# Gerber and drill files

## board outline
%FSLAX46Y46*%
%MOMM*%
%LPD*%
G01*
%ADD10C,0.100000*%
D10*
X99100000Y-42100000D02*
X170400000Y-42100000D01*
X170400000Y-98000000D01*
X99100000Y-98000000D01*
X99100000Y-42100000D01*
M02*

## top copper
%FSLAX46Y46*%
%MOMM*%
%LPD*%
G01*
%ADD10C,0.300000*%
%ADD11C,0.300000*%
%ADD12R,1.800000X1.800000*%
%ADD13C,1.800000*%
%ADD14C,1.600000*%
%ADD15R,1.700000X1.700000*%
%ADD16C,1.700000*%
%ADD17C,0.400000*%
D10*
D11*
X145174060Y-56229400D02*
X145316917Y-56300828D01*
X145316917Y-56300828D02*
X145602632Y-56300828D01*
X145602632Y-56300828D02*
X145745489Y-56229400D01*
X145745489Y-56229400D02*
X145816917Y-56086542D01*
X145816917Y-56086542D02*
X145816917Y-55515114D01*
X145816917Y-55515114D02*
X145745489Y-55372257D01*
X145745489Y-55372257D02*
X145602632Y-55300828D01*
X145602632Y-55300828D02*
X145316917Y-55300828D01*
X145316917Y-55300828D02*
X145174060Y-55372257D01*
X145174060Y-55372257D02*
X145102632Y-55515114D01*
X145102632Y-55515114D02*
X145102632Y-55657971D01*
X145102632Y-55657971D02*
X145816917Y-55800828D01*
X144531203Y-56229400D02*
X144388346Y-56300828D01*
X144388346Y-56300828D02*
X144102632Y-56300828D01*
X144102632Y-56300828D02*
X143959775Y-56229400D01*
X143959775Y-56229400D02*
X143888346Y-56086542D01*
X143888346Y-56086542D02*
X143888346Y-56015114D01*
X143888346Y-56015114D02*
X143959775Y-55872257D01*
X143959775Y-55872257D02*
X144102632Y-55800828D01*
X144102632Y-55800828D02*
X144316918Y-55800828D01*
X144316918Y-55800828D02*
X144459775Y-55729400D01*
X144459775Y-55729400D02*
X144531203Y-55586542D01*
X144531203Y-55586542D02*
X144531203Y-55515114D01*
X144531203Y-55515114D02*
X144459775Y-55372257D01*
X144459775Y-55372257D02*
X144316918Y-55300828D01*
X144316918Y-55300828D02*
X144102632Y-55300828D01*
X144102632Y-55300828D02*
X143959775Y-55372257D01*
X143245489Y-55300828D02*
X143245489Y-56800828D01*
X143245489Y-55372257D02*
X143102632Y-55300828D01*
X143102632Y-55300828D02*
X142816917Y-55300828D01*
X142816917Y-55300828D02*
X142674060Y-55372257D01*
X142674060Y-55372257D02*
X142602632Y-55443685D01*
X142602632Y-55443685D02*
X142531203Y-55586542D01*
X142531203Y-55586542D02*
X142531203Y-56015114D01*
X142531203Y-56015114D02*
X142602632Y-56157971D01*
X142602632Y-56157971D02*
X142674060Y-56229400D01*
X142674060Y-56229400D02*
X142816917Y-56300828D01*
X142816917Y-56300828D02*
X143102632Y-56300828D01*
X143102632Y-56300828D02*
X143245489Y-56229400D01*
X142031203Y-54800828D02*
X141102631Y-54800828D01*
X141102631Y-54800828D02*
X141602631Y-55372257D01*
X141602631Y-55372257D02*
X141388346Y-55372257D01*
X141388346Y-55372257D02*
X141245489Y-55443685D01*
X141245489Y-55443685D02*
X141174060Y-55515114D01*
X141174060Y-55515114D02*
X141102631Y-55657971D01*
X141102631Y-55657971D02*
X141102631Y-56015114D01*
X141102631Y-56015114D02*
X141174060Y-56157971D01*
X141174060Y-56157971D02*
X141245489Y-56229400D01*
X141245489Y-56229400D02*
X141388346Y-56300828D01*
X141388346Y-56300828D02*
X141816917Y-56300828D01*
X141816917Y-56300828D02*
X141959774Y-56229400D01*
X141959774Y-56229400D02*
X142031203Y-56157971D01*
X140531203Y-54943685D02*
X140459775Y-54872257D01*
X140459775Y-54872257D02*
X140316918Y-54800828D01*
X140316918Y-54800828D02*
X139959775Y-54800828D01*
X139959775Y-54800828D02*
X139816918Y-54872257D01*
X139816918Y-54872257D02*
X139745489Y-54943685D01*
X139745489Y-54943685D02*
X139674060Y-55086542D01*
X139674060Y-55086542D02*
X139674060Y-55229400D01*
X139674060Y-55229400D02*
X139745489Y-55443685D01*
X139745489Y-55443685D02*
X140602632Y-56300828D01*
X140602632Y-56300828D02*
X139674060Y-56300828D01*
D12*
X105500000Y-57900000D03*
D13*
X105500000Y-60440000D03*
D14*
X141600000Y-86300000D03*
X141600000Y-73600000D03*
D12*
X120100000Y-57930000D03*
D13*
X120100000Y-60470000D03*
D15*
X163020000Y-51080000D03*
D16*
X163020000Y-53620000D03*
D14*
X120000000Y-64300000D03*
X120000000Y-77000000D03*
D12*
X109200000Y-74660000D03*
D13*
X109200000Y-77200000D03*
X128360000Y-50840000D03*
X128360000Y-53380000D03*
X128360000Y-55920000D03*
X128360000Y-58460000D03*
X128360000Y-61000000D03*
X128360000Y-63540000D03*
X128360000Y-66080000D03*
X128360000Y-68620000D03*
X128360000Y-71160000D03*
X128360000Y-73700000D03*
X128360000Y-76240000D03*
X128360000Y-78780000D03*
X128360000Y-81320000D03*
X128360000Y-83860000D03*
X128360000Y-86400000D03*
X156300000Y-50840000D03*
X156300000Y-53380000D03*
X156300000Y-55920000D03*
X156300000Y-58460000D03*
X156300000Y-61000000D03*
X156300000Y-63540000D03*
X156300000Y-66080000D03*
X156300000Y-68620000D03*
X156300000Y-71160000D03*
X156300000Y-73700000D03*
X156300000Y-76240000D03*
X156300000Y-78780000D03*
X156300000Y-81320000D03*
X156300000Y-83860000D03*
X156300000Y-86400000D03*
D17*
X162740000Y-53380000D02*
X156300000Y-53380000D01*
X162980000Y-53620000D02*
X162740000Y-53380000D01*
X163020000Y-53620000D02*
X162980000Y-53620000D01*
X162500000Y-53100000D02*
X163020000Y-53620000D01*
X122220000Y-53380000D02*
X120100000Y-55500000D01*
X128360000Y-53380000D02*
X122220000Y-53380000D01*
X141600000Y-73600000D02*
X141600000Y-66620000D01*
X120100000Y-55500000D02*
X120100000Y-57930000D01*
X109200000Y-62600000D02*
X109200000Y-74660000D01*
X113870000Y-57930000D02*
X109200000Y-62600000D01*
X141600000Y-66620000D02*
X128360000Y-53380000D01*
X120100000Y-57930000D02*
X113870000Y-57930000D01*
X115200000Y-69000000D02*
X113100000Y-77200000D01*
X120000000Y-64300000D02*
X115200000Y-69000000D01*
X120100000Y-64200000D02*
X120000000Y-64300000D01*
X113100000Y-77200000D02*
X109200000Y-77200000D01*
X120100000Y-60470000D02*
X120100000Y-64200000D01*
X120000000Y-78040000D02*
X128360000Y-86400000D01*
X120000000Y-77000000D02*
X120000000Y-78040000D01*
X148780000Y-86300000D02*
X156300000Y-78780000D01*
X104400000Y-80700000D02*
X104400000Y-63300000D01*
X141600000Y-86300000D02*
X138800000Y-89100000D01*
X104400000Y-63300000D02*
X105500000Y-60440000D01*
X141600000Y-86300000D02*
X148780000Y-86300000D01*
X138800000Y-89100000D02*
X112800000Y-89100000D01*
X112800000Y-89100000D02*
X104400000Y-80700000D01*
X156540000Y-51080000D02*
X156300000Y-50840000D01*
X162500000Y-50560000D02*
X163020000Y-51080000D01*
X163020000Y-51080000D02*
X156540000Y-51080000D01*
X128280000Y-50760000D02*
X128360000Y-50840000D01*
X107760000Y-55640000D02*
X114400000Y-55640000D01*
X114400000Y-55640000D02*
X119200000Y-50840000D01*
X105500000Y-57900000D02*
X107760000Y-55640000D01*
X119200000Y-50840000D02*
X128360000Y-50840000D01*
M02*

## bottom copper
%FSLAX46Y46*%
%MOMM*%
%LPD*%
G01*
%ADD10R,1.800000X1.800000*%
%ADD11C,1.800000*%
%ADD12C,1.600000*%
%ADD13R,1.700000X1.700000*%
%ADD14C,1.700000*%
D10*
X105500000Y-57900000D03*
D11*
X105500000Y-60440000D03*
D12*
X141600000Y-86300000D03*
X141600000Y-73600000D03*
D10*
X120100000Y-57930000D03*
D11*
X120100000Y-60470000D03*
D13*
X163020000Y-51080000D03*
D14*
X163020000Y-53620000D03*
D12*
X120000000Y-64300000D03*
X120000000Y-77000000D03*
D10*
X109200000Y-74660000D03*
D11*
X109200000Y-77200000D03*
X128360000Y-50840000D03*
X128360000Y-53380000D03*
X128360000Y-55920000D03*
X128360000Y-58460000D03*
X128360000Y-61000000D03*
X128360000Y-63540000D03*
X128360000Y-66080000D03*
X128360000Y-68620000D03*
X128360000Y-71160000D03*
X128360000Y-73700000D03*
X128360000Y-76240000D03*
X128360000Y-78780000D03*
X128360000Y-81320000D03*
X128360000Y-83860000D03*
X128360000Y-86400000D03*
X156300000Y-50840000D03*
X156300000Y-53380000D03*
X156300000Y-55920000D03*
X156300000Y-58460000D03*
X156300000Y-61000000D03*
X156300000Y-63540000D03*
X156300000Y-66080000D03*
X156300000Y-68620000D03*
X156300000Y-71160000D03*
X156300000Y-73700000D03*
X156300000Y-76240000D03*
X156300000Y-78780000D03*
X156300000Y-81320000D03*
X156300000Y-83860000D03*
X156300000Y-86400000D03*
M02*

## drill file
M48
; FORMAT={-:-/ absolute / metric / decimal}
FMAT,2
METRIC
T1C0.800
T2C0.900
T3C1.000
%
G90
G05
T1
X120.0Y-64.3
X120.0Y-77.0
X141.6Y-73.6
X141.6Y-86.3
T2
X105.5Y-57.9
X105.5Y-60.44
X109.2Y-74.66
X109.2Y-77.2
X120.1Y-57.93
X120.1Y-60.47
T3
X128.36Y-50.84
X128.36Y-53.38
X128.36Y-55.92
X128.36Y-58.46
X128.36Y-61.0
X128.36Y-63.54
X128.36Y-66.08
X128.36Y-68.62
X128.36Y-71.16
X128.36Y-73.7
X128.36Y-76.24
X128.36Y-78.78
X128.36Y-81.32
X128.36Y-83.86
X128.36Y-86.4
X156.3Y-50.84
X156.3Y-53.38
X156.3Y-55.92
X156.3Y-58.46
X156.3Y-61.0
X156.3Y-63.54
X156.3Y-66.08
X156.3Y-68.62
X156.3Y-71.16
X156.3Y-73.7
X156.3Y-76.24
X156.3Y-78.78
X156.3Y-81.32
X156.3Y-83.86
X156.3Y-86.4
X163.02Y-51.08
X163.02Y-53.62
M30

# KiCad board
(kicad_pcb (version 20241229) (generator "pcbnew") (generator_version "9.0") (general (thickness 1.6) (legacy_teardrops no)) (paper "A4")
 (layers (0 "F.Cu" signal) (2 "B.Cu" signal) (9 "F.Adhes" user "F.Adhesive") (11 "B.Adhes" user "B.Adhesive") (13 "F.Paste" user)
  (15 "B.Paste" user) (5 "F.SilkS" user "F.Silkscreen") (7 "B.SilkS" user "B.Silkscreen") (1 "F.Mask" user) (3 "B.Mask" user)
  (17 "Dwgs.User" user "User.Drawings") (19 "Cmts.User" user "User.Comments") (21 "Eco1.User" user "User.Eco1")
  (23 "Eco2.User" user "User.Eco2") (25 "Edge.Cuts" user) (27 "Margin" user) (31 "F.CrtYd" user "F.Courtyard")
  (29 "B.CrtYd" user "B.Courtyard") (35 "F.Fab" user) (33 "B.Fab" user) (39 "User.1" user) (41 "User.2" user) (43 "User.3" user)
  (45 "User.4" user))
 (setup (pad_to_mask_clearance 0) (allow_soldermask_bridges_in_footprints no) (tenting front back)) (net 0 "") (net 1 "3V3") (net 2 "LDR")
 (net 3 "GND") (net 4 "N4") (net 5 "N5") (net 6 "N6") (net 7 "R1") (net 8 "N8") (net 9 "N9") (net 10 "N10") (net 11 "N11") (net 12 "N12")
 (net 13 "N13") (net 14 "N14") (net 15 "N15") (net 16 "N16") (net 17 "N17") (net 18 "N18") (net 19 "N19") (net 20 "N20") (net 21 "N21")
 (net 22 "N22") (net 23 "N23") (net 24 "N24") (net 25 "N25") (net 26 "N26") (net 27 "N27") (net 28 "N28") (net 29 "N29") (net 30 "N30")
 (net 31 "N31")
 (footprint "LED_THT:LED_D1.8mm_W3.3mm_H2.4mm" (layer "F.Cu") (at 105.5 57.9 -90)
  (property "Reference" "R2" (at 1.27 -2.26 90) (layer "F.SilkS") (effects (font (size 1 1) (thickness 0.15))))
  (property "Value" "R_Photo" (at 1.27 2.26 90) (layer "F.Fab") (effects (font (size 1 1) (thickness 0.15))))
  (pad "1" thru_hole rect (at 0 0 270) (size 1.8 1.8) (drill 0.9) (layers "*.Cu" "*.Mask") (remove_unused_layers no) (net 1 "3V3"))
  (pad "2" thru_hole circle (at 2.54 0 270) (size 1.8 1.8) (drill 0.9) (layers "*.Cu" "*.Mask") (remove_unused_layers no) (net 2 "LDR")))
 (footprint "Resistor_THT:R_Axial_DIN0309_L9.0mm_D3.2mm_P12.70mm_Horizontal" (layer "F.Cu") (at 141.6 86.3 90)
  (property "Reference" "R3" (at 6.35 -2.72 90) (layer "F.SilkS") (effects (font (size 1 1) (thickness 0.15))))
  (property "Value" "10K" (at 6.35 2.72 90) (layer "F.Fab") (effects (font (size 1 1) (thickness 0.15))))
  (pad "1" thru_hole circle (at 0 0 90) (size 1.6 1.6) (drill 0.8) (layers "*.Cu" "*.Mask") (remove_unused_layers no) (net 2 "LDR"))
  (pad "2" thru_hole circle (at 12.7 0 90) (size 1.6 1.6) (drill 0.8) (layers "*.Cu" "*.Mask") (remove_unused_layers no) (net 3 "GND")))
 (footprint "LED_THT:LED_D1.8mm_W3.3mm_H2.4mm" (layer "F.Cu") (at 120.1 57.93 -90)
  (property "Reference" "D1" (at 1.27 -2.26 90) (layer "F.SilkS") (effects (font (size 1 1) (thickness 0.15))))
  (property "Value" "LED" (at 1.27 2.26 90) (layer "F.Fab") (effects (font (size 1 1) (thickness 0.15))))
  (pad "1" thru_hole rect (at 0 0 270) (size 1.8 1.8) (drill 0.9) (layers "*.Cu" "*.Mask") (remove_unused_layers no) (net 3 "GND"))
  (pad "2" thru_hole circle (at 2.54 0 270) (size 1.8 1.8) (drill 0.9) (layers "*.Cu" "*.Mask") (remove_unused_layers no) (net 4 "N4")))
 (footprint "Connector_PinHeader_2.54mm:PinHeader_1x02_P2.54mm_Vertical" (layer "F.Cu") (at 163.02 51.08)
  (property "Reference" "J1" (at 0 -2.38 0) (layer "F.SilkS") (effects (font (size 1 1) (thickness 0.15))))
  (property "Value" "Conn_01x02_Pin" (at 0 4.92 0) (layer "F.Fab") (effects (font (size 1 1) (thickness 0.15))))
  (pad "1" thru_hole rect (at 0 0) (size 1.7 1.7) (drill 1) (layers "*.Cu" "*.Mask") (remove_unused_layers no) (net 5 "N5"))
  (pad "2" thru_hole circle (at 0 2.54) (size 1.7 1.7) (drill 1) (layers "*.Cu" "*.Mask") (remove_unused_layers no) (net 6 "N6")))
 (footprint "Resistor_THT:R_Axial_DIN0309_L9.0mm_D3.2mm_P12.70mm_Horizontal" (layer "F.Cu") (at 120 64.3 -90)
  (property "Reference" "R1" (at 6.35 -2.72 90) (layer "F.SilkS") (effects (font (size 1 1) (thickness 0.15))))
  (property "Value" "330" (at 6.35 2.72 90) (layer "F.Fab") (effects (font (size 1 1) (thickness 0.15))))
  (pad "1" thru_hole circle (at 0 0 270) (size 1.6 1.6) (drill 0.8) (layers "*.Cu" "*.Mask") (remove_unused_layers no) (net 4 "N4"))
  (pad "2" thru_hole circle (at 12.7 0 270) (size 1.6 1.6) (drill 0.8) (layers "*.Cu" "*.Mask") (remove_unused_layers no) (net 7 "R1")))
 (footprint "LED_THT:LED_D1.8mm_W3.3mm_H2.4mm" (layer "F.Cu") (at 109.2 74.66 -90)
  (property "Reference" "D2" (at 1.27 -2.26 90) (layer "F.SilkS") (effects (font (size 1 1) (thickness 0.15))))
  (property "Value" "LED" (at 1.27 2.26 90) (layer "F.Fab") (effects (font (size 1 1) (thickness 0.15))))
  (pad "1" thru_hole rect (at 0 0 270) (size 1.8 1.8) (drill 0.9) (layers "*.Cu" "*.Mask") (remove_unused_layers no) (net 3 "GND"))
  (pad "2" thru_hole circle (at 2.54 0 270) (size 1.8 1.8) (drill 0.9) (layers "*.Cu" "*.Mask") (remove_unused_layers no) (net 4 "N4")))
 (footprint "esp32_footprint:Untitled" (layer "F.Cu") (at 143.6 68.62)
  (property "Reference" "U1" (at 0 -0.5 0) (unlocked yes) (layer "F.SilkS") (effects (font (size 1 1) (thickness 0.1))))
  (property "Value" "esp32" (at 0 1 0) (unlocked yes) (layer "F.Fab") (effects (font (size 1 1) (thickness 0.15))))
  (pad "1" thru_hole circle (at -15.24 -17.78) (size 1.8 1.8) (drill 1) (layers "*.Cu" "*.Mask") (remove_unused_layers no) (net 1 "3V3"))
  (pad "2" thru_hole circle (at -15.24 -15.24) (size 1.8 1.8) (drill 1) (layers "*.Cu" "*.Mask") (remove_unused_layers no) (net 3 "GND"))
  (pad "3" thru_hole circle (at -15.24 -12.7) (size 1.8 1.8) (drill 1) (layers "*.Cu" "*.Mask") (remove_unused_layers no) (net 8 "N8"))
  (pad "4" thru_hole circle (at -15.24 -10.16) (size 1.8 1.8) (drill 1) (layers "*.Cu" "*.Mask") (remove_unused_layers no) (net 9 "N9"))
  (pad "5" thru_hole circle (at -15.24 -7.62) (size 1.8 1.8) (drill 1) (layers "*.Cu" "*.Mask") (remove_unused_layers no) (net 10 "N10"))
  (pad "6" thru_hole circle (at -15.24 -5.08) (size 1.8 1.8) (drill 1) (layers "*.Cu" "*.Mask") (remove_unused_layers no) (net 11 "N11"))
  (pad "7" thru_hole circle (at -15.24 -2.54) (size 1.8 1.8) (drill 1) (layers "*.Cu" "*.Mask") (remove_unused_layers no) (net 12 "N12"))
  (pad "8" thru_hole circle (at -15.24 0) (size 1.8 1.8) (drill 1) (layers "*.Cu" "*.Mask") (remove_unused_layers no) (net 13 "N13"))
  (pad "9" thru_hole circle (at -15.24 2.54) (size 1.8 1.8) (drill 1) (layers "*.Cu" "*.Mask") (remove_unused_layers no) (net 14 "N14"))
  (pad "10" thru_hole circle (at -15.24 5.08) (size 1.8 1.8) (drill 1) (layers "*.Cu" "*.Mask") (remove_unused_layers no) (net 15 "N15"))
  (pad "11" thru_hole circle (at -15.24 7.62) (size 1.8 1.8) (drill 1) (layers "*.Cu" "*.Mask") (remove_unused_layers no) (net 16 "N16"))
  (pad "12" thru_hole circle (at -15.24 10.16) (size 1.8 1.8) (drill 1) (layers "*.Cu" "*.Mask") (remove_unused_layers no) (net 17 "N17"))
  (pad "13" thru_hole circle (at -15.24 12.7) (size 1.8 1.8) (drill 1) (layers "*.Cu" "*.Mask") (remove_unused_layers no) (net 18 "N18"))
  (pad "14" thru_hole circle (at -15.24 15.24) (size 1.8 1.8) (drill 1) (layers "*.Cu" "*.Mask") (remove_unused_layers no) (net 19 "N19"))
  (pad "15" thru_hole circle (at -15.24 17.78) (size 1.8 1.8) (drill 1) (layers "*.Cu" "*.Mask") (remove_unused_layers no) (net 7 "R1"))
  (pad "16" thru_hole circle (at 12.7 -17.78) (size 1.8 1.8) (drill 1) (layers "*.Cu" "*.Mask") (remove_unused_layers no) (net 5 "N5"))
  (pad "17" thru_hole circle (at 12.7 -15.24) (size 1.8 1.8) (drill 1) (layers "*.Cu" "*.Mask") (remove_unused_layers no) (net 6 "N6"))
  (pad "18" thru_hole circle (at 12.7 -12.7) (size 1.8 1.8) (drill 1) (layers "*.Cu" "*.Mask") (remove_unused_layers no) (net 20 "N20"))
  (pad "19" thru_hole circle (at 12.7 -10.16) (size 1.8 1.8) (drill 1) (layers "*.Cu" "*.Mask") (remove_unused_layers no) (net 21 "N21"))
  (pad "20" thru_hole circle (at 12.7 -7.62) (size 1.8 1.8) (drill 1) (layers "*.Cu" "*.Mask") (remove_unused_layers no) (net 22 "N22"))
  (pad "21" thru_hole circle (at 12.7 -5.08) (size 1.8 1.8) (drill 1) (layers "*.Cu" "*.Mask") (remove_unused_layers no) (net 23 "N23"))
  (pad "22" thru_hole circle (at 12.7 -2.54) (size 1.8 1.8) (drill 1) (layers "*.Cu" "*.Mask") (remove_unused_layers no) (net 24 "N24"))
  (pad "23" thru_hole circle (at 12.7 0) (size 1.8 1.8) (drill 1) (layers "*.Cu" "*.Mask") (remove_unused_layers no) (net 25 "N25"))
  (pad "24" thru_hole circle (at 12.7 2.54) (size 1.8 1.8) (drill 1) (layers "*.Cu" "*.Mask") (remove_unused_layers no) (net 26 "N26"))
  (pad "25" thru_hole circle (at 12.7 5.08) (size 1.8 1.8) (drill 1) (layers "*.Cu" "*.Mask") (remove_unused_layers no) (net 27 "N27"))
  (pad "26" thru_hole circle (at 12.7 7.62) (size 1.8 1.8) (drill 1) (layers "*.Cu" "*.Mask") (remove_unused_layers no) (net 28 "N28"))
  (pad "27" thru_hole circle (at 12.7 10.16) (size 1.8 1.8) (drill 1) (layers "*.Cu" "*.Mask") (remove_unused_layers no) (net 2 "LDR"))
  (pad "28" thru_hole circle (at 12.7 12.7) (size 1.8 1.8) (drill 1) (layers "*.Cu" "*.Mask") (remove_unused_layers no) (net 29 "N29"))
  (pad "29" thru_hole circle (at 12.7 15.24) (size 1.8 1.8) (drill 1) (layers "*.Cu" "*.Mask") (remove_unused_layers no) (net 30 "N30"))
  (pad "30" thru_hole circle (at 12.7 17.78) (size 1.8 1.8) (drill 1) (layers "*.Cu" "*.Mask") (remove_unused_layers no) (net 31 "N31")))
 (gr_rect (start 99.1 42.1) (end 170.4 98) (stroke (width 0.1) (type solid)) (fill no) (layer "Edge.Cuts"))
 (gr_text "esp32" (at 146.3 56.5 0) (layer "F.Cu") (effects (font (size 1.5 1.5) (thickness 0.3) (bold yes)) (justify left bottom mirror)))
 (segment (start 162.74 53.38) (end 156.3 53.38) (width 0.4) (layer "F.Cu") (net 6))
 (segment (start 162.98 53.62) (end 162.74 53.38) (width 0.4) (layer "F.Cu") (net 6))
 (segment (start 163.02 53.62) (end 162.98 53.62) (width 0.4) (layer "F.Cu") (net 6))
 (segment (start 162.5 53.1) (end 163.02 53.62) (width 0.4) (layer "F.Cu") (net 6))
 (segment (start 122.22 53.38) (end 120.1 55.5) (width 0.4) (layer "F.Cu") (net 3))
 (segment (start 128.36 53.38) (end 122.22 53.38) (width 0.4) (layer "F.Cu") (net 3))
 (segment (start 141.6 73.6) (end 141.6 66.62) (width 0.4) (layer "F.Cu") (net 3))
 (segment (start 120.1 55.5) (end 120.1 57.93) (width 0.4) (layer "F.Cu") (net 3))
 (segment (start 109.2 62.6) (end 109.2 74.66) (width 0.4) (layer "F.Cu") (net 3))
 (segment (start 113.87 57.93) (end 109.2 62.6) (width 0.4) (layer "F.Cu") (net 3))
 (segment (start 141.6 66.62) (end 128.36 53.38) (width 0.4) (layer "F.Cu") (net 3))
 (segment (start 120.1 57.93) (end 113.87 57.93) (width 0.4) (layer "F.Cu") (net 3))
 (segment (start 115.2 69) (end 113.1 77.2) (width 0.4) (layer "F.Cu") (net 4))
 (segment (start 120 64.3) (end 115.2 69) (width 0.4) (layer "F.Cu") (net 4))
 (segment (start 120.1 64.2) (end 120 64.3) (width 0.4) (layer "F.Cu") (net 4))
 (segment (start 113.1 77.2) (end 109.2 77.2) (width 0.4) (layer "F.Cu") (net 4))
 (segment (start 120.1 60.47) (end 120.1 64.2) (width 0.4) (layer "F.Cu") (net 4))
 (segment (start 120 78.04) (end 128.36 86.4) (width 0.4) (layer "F.Cu") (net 7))
 (segment (start 120 77) (end 120 78.04) (width 0.4) (layer "F.Cu") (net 7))
 (segment (start 148.78 86.3) (end 156.3 78.78) (width 0.4) (layer "F.Cu") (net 2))
 (segment (start 104.4 80.7) (end 104.4 63.3) (width 0.4) (layer "F.Cu") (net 2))
 (segment (start 141.6 86.3) (end 138.8 89.1) (width 0.4) (layer "F.Cu") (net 2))
 (segment (start 104.4 63.3) (end 105.5 60.44) (width 0.4) (layer "F.Cu") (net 2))
 (segment (start 141.6 86.3) (end 148.78 86.3) (width 0.4) (layer "F.Cu") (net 2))
 (segment (start 138.8 89.1) (end 112.8 89.1) (width 0.4) (layer "F.Cu") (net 2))
 (segment (start 112.8 89.1) (end 104.4 80.7) (width 0.4) (layer "F.Cu") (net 2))
 (segment (start 156.54 51.08) (end 156.3 50.84) (width 0.4) (layer "F.Cu") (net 5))
 (segment (start 162.5 50.56) (end 163.02 51.08) (width 0.4) (layer "F.Cu") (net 5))
 (segment (start 163.02 51.08) (end 156.54 51.08) (width 0.4) (layer "F.Cu") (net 5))
 (segment (start 128.28 50.76) (end 128.36 50.84) (width 0.4) (layer "F.Cu") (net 1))
 (segment (start 107.76 55.64) (end 114.4 55.64) (width 0.4) (layer "F.Cu") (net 1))
 (segment (start 114.4 55.64) (end 119.2 50.84) (width 0.4) (layer "F.Cu") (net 1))
 (segment (start 105.5 57.9) (end 107.76 55.64) (width 0.4) (layer "F.Cu") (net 1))
 (segment (start 119.2 50.84) (end 128.36 50.84) (width 0.4) (layer "F.Cu") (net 1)))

